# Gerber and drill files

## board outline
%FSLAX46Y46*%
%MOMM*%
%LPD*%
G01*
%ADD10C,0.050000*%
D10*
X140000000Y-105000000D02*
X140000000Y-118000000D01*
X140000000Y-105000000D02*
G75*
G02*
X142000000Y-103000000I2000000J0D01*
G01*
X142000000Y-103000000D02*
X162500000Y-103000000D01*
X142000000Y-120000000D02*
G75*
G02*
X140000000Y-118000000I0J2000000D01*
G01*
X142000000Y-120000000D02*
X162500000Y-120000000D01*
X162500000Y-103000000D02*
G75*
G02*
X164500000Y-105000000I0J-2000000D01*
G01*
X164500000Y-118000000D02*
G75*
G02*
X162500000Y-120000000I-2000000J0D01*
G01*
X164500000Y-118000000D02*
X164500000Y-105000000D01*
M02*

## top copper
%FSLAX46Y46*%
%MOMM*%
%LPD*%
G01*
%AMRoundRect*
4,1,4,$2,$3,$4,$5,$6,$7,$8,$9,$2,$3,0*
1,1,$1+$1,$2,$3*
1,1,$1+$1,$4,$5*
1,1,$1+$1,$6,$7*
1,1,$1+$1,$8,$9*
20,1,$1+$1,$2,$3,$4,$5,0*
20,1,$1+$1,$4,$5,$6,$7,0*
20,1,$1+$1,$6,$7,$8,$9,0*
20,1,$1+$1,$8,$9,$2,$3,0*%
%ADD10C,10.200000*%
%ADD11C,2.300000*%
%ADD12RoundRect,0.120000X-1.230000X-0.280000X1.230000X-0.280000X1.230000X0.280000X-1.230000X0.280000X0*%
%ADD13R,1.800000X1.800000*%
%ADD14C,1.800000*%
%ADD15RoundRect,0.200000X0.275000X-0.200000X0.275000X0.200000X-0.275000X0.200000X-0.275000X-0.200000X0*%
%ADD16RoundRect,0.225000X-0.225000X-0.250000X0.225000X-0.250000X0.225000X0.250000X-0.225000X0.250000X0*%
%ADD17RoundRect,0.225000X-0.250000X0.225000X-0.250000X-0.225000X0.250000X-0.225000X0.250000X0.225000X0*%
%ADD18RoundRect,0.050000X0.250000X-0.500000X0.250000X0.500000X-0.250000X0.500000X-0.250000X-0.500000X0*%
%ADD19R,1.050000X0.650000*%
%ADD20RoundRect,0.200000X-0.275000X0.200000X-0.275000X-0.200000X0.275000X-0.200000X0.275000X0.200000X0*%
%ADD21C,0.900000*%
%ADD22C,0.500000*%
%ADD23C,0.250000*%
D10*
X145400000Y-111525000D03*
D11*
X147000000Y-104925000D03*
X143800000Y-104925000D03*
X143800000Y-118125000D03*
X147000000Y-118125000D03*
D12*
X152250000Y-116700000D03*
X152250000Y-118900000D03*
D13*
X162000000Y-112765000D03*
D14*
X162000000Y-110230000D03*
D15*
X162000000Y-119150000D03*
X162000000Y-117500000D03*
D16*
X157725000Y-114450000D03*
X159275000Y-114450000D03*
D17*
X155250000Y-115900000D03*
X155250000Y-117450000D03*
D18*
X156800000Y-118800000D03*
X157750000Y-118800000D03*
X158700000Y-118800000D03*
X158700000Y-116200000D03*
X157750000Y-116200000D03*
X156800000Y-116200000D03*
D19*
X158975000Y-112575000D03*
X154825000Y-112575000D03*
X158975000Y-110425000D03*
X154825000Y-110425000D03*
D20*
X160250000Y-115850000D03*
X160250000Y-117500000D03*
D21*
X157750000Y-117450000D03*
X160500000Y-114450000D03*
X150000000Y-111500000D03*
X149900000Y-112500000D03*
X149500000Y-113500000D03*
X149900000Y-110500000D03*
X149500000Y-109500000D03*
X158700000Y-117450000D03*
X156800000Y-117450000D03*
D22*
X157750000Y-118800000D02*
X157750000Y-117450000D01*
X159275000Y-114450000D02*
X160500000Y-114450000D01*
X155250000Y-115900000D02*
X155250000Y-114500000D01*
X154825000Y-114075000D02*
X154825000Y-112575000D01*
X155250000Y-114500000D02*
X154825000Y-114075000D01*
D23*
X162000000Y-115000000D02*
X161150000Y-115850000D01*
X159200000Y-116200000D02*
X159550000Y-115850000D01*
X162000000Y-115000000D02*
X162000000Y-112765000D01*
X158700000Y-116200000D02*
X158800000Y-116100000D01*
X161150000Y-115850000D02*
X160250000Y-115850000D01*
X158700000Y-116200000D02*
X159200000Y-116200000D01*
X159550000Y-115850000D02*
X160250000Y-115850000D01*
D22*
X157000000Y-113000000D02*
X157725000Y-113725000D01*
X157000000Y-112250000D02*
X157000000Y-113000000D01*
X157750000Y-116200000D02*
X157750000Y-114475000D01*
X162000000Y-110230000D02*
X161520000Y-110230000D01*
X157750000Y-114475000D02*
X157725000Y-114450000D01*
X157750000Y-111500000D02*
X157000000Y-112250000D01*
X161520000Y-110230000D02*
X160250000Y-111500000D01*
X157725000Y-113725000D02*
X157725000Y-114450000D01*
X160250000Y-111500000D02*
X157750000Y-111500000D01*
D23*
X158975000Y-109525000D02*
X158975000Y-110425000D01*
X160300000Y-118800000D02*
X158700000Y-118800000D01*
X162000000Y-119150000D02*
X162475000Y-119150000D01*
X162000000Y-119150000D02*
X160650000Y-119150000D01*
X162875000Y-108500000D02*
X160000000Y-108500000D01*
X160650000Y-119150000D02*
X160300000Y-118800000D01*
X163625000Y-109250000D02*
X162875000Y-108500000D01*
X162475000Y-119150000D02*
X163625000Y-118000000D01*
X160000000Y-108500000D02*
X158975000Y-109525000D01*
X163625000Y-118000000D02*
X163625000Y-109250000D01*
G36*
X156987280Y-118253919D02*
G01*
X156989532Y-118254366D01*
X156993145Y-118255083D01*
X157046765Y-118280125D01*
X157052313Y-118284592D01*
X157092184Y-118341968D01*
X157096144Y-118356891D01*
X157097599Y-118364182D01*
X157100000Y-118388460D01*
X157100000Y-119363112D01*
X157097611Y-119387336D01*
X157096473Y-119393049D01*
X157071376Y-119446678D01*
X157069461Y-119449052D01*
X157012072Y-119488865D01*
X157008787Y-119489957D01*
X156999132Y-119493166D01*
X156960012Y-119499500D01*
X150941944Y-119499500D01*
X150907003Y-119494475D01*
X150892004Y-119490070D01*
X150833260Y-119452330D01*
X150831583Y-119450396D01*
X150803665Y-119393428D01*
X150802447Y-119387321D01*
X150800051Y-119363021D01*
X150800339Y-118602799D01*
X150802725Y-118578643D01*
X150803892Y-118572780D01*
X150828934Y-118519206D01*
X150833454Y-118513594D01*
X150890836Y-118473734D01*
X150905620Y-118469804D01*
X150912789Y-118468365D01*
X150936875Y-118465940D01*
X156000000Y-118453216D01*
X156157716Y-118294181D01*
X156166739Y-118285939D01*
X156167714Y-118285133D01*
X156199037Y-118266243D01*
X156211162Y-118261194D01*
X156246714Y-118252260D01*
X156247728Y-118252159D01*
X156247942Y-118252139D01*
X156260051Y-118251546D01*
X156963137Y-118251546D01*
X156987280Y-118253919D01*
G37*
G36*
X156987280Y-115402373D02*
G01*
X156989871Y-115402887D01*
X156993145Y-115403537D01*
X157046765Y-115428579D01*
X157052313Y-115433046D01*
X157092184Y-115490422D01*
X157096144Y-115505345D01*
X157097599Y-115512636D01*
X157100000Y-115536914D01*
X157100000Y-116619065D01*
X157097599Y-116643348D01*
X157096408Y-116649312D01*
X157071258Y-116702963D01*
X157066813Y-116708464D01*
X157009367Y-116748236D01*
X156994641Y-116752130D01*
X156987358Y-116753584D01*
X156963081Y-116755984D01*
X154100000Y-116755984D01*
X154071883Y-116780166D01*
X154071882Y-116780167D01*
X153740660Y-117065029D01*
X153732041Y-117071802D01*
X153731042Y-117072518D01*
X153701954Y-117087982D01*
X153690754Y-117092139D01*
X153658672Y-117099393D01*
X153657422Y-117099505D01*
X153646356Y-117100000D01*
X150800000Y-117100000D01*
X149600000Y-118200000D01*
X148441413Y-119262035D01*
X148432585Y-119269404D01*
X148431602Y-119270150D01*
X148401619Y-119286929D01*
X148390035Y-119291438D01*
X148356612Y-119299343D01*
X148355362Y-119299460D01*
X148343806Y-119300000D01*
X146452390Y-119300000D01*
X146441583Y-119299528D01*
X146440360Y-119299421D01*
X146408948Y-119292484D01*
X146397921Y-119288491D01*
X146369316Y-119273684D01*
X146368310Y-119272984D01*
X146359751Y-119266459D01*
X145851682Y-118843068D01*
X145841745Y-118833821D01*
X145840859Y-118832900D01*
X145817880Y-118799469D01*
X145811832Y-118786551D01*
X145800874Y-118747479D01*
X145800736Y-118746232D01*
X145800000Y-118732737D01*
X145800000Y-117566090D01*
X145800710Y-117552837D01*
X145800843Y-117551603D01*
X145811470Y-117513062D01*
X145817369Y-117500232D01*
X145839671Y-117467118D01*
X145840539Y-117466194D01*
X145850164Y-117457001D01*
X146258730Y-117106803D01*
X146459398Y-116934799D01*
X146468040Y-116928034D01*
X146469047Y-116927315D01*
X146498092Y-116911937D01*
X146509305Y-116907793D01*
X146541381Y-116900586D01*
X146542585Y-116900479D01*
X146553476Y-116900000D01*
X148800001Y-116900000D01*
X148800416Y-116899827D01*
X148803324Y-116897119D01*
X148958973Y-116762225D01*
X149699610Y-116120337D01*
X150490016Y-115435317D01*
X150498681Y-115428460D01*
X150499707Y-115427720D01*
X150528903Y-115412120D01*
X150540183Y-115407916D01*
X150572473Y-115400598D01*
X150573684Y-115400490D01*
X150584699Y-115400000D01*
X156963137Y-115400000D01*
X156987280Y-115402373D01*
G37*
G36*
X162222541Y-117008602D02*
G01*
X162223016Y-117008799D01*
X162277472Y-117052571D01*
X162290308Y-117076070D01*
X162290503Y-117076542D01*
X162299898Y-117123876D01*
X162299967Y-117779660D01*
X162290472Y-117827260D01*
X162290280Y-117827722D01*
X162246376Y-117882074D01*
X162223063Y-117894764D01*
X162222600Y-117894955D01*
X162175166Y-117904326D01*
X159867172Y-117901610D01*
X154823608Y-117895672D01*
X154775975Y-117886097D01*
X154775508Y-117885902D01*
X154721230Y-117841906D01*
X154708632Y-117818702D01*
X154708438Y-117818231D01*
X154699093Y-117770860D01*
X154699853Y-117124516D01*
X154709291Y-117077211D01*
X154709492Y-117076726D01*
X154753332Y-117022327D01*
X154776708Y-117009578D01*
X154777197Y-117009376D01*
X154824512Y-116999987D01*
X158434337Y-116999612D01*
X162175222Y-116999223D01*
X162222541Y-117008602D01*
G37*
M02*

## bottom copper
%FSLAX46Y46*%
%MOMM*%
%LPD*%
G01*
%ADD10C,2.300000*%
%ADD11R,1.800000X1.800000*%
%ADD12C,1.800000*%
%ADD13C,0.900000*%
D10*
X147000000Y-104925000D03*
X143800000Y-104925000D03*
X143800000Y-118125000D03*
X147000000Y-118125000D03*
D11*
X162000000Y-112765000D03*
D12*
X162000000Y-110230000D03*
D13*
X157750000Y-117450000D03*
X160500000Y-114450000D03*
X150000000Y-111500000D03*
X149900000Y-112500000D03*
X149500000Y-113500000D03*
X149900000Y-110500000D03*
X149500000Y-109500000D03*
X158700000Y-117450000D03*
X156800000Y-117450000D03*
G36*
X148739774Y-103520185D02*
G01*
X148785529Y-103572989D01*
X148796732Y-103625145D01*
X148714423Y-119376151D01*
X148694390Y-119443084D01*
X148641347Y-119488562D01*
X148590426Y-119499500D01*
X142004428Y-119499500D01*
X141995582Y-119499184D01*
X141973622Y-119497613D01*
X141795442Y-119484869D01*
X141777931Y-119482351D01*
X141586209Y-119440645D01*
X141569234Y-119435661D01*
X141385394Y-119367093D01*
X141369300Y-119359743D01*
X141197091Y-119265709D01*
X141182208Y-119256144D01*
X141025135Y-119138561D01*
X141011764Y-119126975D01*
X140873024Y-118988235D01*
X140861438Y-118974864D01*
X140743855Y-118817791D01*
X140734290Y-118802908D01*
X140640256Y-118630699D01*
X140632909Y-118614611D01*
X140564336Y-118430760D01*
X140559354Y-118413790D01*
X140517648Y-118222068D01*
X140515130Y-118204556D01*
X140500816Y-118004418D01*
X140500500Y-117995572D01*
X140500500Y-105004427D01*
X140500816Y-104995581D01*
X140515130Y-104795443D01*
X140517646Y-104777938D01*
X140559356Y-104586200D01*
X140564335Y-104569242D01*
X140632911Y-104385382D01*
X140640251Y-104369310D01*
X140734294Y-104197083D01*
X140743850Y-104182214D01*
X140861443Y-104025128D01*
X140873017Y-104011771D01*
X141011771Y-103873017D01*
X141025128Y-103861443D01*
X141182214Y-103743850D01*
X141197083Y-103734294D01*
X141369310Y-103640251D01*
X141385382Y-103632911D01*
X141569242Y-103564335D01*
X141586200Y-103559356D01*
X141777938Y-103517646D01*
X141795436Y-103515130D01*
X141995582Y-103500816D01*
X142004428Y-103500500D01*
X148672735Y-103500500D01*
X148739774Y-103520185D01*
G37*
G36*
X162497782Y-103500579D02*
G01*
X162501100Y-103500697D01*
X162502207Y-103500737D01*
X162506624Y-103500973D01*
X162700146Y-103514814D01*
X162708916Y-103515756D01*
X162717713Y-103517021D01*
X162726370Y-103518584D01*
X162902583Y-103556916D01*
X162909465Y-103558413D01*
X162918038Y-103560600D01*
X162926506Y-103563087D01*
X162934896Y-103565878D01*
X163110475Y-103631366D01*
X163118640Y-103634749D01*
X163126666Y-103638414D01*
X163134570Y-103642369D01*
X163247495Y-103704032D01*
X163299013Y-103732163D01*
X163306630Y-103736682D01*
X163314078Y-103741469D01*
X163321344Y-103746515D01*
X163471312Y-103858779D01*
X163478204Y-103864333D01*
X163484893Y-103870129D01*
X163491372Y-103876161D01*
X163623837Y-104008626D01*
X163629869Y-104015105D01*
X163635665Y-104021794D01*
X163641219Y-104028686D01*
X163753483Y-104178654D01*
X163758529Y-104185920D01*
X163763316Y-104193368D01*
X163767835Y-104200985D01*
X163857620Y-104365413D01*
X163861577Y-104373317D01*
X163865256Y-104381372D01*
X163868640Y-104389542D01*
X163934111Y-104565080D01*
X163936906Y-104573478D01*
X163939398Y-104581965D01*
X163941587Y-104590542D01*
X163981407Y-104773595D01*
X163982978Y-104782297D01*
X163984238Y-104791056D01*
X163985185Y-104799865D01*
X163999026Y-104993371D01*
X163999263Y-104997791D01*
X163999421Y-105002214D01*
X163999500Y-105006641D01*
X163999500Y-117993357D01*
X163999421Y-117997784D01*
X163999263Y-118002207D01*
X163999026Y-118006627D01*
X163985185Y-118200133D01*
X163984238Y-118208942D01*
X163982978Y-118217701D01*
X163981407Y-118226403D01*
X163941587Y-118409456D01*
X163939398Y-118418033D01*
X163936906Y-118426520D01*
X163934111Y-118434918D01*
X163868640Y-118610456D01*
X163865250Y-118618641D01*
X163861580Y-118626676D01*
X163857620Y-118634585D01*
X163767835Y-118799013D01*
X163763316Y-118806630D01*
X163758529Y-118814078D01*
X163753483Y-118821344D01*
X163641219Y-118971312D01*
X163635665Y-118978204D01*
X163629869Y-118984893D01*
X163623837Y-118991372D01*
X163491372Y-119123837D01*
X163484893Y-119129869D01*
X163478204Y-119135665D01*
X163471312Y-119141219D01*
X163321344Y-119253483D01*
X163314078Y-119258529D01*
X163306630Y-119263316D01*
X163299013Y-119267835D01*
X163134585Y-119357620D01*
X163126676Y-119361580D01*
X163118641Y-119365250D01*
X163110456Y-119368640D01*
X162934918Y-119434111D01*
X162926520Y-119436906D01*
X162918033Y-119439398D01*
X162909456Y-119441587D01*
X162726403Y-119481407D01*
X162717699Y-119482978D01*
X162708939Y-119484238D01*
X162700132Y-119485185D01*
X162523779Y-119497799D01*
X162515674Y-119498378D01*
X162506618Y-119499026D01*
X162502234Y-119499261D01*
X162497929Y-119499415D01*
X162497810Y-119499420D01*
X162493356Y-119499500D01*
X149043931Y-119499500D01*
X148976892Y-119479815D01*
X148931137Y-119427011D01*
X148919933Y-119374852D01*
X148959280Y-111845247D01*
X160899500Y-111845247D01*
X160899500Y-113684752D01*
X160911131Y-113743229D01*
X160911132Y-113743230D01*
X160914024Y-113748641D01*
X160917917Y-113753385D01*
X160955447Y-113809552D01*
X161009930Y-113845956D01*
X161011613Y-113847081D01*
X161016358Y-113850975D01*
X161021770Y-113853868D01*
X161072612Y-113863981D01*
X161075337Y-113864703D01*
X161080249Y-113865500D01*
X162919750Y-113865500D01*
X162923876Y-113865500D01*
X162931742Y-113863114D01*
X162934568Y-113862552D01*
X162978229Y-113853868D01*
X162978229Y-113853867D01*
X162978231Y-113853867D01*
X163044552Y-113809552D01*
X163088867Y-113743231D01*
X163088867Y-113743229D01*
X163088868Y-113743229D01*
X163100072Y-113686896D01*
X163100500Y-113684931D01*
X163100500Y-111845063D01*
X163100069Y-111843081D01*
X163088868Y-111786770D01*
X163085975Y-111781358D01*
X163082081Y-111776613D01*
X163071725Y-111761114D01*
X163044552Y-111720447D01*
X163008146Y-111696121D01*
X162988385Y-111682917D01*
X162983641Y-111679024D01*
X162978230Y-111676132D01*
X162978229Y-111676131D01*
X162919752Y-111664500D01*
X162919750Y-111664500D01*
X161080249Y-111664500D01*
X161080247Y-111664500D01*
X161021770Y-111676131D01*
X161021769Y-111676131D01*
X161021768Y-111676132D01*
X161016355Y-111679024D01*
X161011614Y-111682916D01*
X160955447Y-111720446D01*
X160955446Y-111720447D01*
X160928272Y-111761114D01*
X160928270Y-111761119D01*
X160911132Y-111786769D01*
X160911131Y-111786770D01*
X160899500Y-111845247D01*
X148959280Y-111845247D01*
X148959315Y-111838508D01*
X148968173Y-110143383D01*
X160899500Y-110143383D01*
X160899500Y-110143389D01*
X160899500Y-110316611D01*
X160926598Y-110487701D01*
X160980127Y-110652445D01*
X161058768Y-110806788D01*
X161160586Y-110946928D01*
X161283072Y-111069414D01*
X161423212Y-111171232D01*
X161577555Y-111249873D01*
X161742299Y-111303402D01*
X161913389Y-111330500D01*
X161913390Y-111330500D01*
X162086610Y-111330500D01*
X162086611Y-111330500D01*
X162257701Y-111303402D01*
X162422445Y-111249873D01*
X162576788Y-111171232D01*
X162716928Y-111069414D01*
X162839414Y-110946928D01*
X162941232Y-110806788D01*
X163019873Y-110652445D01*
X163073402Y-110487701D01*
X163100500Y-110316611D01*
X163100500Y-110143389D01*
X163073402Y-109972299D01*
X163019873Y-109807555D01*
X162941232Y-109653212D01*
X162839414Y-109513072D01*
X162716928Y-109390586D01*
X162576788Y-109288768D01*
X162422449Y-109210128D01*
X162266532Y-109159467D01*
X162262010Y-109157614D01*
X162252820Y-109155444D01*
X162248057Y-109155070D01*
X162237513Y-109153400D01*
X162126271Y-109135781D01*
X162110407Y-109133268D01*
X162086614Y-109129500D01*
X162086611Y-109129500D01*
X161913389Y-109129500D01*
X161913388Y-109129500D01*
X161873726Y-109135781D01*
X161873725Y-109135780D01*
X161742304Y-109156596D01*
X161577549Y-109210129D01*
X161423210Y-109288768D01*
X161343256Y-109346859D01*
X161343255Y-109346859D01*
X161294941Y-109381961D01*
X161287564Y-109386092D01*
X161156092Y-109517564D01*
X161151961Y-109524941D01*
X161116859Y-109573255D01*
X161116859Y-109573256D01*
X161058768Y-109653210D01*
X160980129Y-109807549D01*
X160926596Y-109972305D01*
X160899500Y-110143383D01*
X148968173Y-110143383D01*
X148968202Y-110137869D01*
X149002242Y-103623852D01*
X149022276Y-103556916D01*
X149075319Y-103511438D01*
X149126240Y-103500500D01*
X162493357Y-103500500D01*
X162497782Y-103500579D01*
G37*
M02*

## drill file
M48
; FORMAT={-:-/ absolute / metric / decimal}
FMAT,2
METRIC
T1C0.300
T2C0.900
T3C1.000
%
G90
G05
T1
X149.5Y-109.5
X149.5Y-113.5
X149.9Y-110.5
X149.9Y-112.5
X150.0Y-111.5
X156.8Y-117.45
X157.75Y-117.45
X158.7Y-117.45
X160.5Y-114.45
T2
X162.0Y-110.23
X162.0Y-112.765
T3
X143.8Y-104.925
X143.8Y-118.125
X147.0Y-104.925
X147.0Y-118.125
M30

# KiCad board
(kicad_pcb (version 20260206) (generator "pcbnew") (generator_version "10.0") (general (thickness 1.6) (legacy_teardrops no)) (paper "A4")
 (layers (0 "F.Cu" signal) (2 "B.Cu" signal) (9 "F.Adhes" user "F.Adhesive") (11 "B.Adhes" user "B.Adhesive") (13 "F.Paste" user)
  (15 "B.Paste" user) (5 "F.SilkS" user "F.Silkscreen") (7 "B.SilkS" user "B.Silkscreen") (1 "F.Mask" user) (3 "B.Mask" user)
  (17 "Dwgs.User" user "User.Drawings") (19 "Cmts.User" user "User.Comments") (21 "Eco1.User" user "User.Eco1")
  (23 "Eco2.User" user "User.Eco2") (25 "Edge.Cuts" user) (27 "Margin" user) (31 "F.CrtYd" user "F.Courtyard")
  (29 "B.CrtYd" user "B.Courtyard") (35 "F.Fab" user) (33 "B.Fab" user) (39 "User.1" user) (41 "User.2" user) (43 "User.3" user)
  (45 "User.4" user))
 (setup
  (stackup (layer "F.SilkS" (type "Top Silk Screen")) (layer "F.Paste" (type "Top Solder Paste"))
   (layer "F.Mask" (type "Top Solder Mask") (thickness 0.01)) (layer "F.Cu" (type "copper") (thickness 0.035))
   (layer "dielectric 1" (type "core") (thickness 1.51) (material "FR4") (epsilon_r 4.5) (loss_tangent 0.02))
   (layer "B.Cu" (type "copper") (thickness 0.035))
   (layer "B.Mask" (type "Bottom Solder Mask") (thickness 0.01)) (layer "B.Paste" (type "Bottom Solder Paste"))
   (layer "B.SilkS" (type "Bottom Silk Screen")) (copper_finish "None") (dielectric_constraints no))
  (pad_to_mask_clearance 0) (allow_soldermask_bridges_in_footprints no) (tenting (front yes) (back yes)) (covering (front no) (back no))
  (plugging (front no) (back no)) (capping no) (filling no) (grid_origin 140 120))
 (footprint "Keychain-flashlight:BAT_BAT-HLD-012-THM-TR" (layer "F.Cu") (at 145.4 111.525 -90)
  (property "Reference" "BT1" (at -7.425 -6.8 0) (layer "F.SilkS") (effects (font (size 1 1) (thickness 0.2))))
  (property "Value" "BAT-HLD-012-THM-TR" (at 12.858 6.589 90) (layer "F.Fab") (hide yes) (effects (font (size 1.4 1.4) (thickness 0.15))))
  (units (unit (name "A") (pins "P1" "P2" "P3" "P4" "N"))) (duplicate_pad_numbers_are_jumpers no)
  (pad "N" smd circle (at 0 0 270) (size 10.2 10.2) (layers "F.Cu" "F.Mask") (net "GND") (solder_mask_margin 0.102))
  (pad "P1" thru_hole circle (at -6.6 -1.6 270) (size 2.3 2.3) (drill 1) (layers "*.Cu" "*.Mask") (remove_unused_layers no) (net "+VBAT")
   (solder_mask_margin 0.102))
  (pad "P2" thru_hole circle (at -6.6 1.6 270) (size 2.3 2.3) (drill 1) (layers "*.Cu" "*.Mask") (remove_unused_layers no) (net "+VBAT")
   (solder_mask_margin 0.102))
  (pad "P3" thru_hole circle (at 6.6 1.6 270) (size 2.3 2.3) (drill 1) (layers "*.Cu" "*.Mask") (remove_unused_layers no) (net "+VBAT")
   (solder_mask_margin 0.102))
  (pad "P4" thru_hole circle (at 6.6 -1.6 270) (size 2.3 2.3) (drill 1) (layers "*.Cu" "*.Mask") (remove_unused_layers no) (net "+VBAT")
   (solder_mask_margin 0.102)))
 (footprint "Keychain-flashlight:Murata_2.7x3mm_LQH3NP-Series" (layer "F.Cu") (at 152.25 117.8 -90)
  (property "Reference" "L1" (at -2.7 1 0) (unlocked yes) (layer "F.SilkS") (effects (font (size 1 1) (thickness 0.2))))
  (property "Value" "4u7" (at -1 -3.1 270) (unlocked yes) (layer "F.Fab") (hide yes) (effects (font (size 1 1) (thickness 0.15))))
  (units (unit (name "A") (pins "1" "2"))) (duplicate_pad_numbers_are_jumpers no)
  (pad "1" smd roundrect (at -1.1 0) (size 2.7 0.8) (layers "F.Cu" "F.Mask" "F.Paste") (roundrect_rratio 0.15) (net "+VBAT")
   (thermal_bridge_angle 45))
  (pad "2" smd roundrect (at 1.1 0) (size 2.7 0.8) (layers "F.Cu" "F.Mask" "F.Paste") (roundrect_rratio 0.15) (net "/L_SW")
   (thermal_bridge_angle 45)))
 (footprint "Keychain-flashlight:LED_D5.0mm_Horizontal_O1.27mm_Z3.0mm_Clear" (layer "F.Cu") (at 162 112.77 90)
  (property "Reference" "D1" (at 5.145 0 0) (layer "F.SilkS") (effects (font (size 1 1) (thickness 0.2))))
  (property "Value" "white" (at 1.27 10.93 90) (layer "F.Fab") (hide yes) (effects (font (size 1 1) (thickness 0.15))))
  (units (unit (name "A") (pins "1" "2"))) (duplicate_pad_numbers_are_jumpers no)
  (pad "1" thru_hole rect (at 0.005 0 90) (size 1.8 1.8) (drill 0.9) (layers "*.Cu" "*.Mask") (remove_unused_layers no) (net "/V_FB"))
  (pad "2" thru_hole circle (at 2.54 0 90) (size 1.8 1.8) (drill 0.9) (layers "*.Cu" "*.Mask") (remove_unused_layers no) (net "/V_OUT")))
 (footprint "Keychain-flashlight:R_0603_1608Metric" (layer "F.Cu") (at 162 118.325 90)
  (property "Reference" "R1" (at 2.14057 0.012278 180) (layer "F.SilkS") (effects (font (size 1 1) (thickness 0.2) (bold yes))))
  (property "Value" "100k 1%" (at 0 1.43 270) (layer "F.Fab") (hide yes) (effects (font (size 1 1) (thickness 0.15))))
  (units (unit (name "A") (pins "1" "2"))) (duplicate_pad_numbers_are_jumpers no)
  (pad "1" smd roundrect (at -0.825 0 90) (size 0.8 0.95) (layers "F.Cu" "F.Mask" "F.Paste") (roundrect_rratio 0.25) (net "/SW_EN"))
  (pad "2" smd roundrect (at 0.825 0 90) (size 0.8 0.95) (layers "F.Cu" "F.Mask" "F.Paste") (roundrect_rratio 0.25) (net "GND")))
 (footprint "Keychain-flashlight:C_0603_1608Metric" (layer "F.Cu") (at 158.5 114.45)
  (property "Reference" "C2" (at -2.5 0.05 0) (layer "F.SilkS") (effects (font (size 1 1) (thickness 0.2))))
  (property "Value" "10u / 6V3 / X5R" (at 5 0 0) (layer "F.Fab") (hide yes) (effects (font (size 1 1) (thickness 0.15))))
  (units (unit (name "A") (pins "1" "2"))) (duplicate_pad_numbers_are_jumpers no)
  (pad "1" smd roundrect (at -0.775 0) (size 0.9 0.95) (layers "F.Cu" "F.Mask" "F.Paste") (roundrect_rratio 0.25) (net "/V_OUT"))
  (pad "2" smd roundrect (at 0.775 0) (size 0.9 0.95) (layers "F.Cu" "F.Mask" "F.Paste") (roundrect_rratio 0.25) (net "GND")))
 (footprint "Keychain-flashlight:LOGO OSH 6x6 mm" (layer "F.Cu") (at 157.498962 106.370917)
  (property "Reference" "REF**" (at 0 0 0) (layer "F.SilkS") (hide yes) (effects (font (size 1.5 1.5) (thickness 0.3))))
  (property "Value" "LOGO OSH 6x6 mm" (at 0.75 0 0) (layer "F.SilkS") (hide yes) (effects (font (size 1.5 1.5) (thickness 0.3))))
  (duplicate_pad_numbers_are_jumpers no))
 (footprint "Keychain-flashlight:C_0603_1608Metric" (layer "F.Cu") (at 155.25 116.675 -90)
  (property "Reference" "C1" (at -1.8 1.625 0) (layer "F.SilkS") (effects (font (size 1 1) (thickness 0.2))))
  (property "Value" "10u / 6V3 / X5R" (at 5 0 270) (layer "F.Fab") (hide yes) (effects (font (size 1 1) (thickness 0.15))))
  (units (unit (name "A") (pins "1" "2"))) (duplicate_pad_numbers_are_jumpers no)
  (pad "1" smd roundrect (at -0.775 0 270) (size 0.9 0.95) (layers "F.Cu" "F.Mask" "F.Paste") (roundrect_rratio 0.25) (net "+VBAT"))
  (pad "2" smd roundrect (at 0.775 0 270) (size 0.9 0.95) (layers "F.Cu" "F.Mask" "F.Paste") (roundrect_rratio 0.25) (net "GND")))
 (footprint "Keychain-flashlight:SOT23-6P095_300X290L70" (layer "F.Cu") (at 157.75 117.5 90)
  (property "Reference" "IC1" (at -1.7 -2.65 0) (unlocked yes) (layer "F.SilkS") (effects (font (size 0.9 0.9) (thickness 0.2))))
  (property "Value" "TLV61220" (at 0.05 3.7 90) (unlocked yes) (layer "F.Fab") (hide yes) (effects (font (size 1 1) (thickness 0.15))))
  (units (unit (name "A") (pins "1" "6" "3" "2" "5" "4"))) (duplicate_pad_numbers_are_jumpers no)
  (pad "1" smd roundrect (at -1.3 -0.95 90) (size 1.1 0.6) (layers "F.Cu" "F.Mask" "F.Paste") (roundrect_rratio 0.08333333333) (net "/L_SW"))
  (pad "2" smd roundrect (at -1.3 0 90) (size 1.1 0.6) (layers "F.Cu" "F.Mask" "F.Paste") (roundrect_rratio 0.08333333333) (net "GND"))
  (pad "3" smd roundrect (at -1.3 0.95 90) (size 1.1 0.6) (layers "F.Cu" "F.Mask" "F.Paste") (roundrect_rratio 0.08333333333) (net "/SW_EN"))
  (pad "4" smd roundrect (at 1.3 0.95 90) (size 1.1 0.6) (layers "F.Cu" "F.Mask" "F.Paste") (roundrect_rratio 0.08333333333) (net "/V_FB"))
  (pad "5" smd roundrect (at 1.3 0 90) (size 1.1 0.6) (layers "F.Cu" "F.Mask" "F.Paste") (roundrect_rratio 0.08333333333) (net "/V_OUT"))
  (pad "6" smd roundrect (at 1.3 -0.95 90) (size 1.1 0.6) (layers "F.Cu" "F.Mask" "F.Paste") (roundrect_rratio 0.08333333333) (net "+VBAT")))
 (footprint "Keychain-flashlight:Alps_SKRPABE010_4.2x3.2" (layer "F.Cu") (at 156.9 111.5 180)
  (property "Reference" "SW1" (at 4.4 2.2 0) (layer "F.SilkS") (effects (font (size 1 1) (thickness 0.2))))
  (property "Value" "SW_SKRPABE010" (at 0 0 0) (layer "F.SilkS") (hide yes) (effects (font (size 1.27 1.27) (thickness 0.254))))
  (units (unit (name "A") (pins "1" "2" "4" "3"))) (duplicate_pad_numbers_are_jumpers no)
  (pad "1" smd rect (at -2.075 -1.075 270) (size 0.65 1.05) (layers "F.Cu" "F.Mask" "F.Paste") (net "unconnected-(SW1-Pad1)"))
  (pad "2" smd rect (at 2.075 -1.075 270) (size 0.65 1.05) (layers "F.Cu" "F.Mask" "F.Paste") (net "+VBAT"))
  (pad "3" smd rect (at -2.075 1.075 270) (size 0.65 1.05) (layers "F.Cu" "F.Mask" "F.Paste") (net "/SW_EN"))
  (pad "4" smd rect (at 2.075 1.075 270) (size 0.65 1.05) (layers "F.Cu" "F.Mask" "F.Paste") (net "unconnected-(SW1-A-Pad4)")))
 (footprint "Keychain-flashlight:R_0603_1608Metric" (layer "F.Cu") (at 160.25 116.675 -90)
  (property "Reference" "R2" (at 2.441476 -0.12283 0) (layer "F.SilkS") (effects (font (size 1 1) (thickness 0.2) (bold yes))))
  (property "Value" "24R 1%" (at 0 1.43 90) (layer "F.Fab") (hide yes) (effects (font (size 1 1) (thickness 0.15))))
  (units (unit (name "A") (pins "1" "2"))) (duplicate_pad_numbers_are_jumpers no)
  (pad "1" smd roundrect (at -0.825 0 270) (size 0.8 0.95) (layers "F.Cu" "F.Mask" "F.Paste") (roundrect_rratio 0.25) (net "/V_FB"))
  (pad "2" smd roundrect (at 0.825 0 270) (size 0.8 0.95) (layers "F.Cu" "F.Mask" "F.Paste") (roundrect_rratio 0.25) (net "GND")))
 (gr_line (start 140 105) (end 140 118) (stroke (width 0.05) (type default)) (layer "Edge.Cuts"))
 (gr_arc (start 140 105) (mid 140.585786 103.585786) (end 142 103) (stroke (width 0.05) (type default)) (layer "Edge.Cuts"))
 (gr_line (start 142 103) (end 162.5 103) (stroke (width 0.05) (type default)) (layer "Edge.Cuts"))
 (gr_arc (start 142 120) (mid 140.585786 119.414214) (end 140 118) (stroke (width 0.05) (type default)) (layer "Edge.Cuts"))
 (gr_line (start 142 120) (end 162.5 120) (stroke (width 0.05) (type default)) (layer "Edge.Cuts"))
 (gr_arc (start 162.5 103) (mid 163.914214 103.585786) (end 164.5 105) (stroke (width 0.05) (type default)) (layer "Edge.Cuts"))
 (gr_arc (start 164.5 118) (mid 163.914214 119.414214) (end 162.5 120) (stroke (width 0.05) (type default)) (layer "Edge.Cuts"))
 (gr_line (start 164.5 118) (end 164.5 105) (stroke (width 0.05) (type default)) (layer "Edge.Cuts"))
 (segment (start 157.75 118.8) (end 157.75 117.45) (width 0.5) (layer "F.Cu") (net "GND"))
 (segment (start 159.275 114.45) (end 160.5 114.45) (width 0.5) (layer "F.Cu") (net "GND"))
 (via (at 157.75 117.45) (size 0.9) (drill 0.3) (layers "F.Cu" "B.Cu") (free yes) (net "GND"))
 (via (at 160.5 114.45) (size 0.9) (drill 0.3) (layers "F.Cu" "B.Cu") (free yes) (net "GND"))
 (via (at 150 111.5) (size 0.9) (drill 0.3) (layers "F.Cu" "B.Cu") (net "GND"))
 (via (at 149.9 112.5) (size 0.9) (drill 0.3) (layers "F.Cu" "B.Cu") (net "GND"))
 (via (at 149.5 113.5) (size 0.9) (drill 0.3) (layers "F.Cu" "B.Cu") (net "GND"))
 (via (at 149.9 110.5) (size 0.9) (drill 0.3) (layers "F.Cu" "B.Cu") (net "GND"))
 (via (at 149.5 109.5) (size 0.9) (drill 0.3) (layers "F.Cu" "B.Cu") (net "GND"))
 (via (at 158.7 117.45) (size 0.9) (drill 0.3) (layers "F.Cu" "B.Cu") (free yes) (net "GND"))
 (via (at 156.8 117.45) (size 0.9) (drill 0.3) (layers "F.Cu" "B.Cu") (free yes) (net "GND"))
 (segment (start 155.25 115.9) (end 155.25 114.5) (width 0.5) (layer "F.Cu") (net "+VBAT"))
 (segment (start 154.825 114.075) (end 154.825 112.575) (width 0.5) (layer "F.Cu") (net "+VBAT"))
 (segment (start 155.25 114.5) (end 154.825 114.075) (width 0.5) (layer "F.Cu") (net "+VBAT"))
 (segment (start 162 115) (end 161.15 115.85) (width 0.25) (layer "F.Cu") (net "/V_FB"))
 (segment (start 159.2 116.2) (end 159.55 115.85) (width 0.25) (layer "F.Cu") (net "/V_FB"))
 (segment (start 162 115) (end 162 112.765) (width 0.25) (layer "F.Cu") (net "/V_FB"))
 (segment (start 158.7 116.2) (end 158.8 116.1) (width 0.25) (layer "F.Cu") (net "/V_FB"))
 (segment (start 161.15 115.85) (end 160.25 115.85) (width 0.25) (layer "F.Cu") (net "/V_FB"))
 (segment (start 158.7 116.2) (end 159.2 116.2) (width 0.25) (layer "F.Cu") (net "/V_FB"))
 (segment (start 159.55 115.85) (end 160.25 115.85) (width 0.25) (layer "F.Cu") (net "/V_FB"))
 (segment (start 157 113) (end 157.725 113.725) (width 0.5) (layer "F.Cu") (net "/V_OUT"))
 (segment (start 157 112.25) (end 157 113) (width 0.5) (layer "F.Cu") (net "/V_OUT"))
 (segment (start 157.75 116.2) (end 157.75 114.475) (width 0.5) (layer "F.Cu") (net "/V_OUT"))
 (segment (start 162 110.23) (end 161.52 110.23) (width 0.5) (layer "F.Cu") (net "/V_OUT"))
 (segment (start 157.75 114.475) (end 157.725 114.45) (width 0.5) (layer "F.Cu") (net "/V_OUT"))
 (segment (start 157.75 111.5) (end 157 112.25) (width 0.5) (layer "F.Cu") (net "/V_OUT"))
 (segment (start 161.52 110.23) (end 160.25 111.5) (width 0.5) (layer "F.Cu") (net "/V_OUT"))
 (segment (start 157.725 113.725) (end 157.725 114.45) (width 0.5) (layer "F.Cu") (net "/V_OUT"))
 (segment (start 160.25 111.5) (end 157.75 111.5) (width 0.5) (layer "F.Cu") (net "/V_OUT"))
 (segment (start 158.975 109.525) (end 158.975 110.425) (width 0.25) (layer "F.Cu") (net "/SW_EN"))
 (segment (start 160.3 118.8) (end 158.7 118.8) (width 0.25) (layer "F.Cu") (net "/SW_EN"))
 (segment (start 162 119.15) (end 162.475 119.15) (width 0.25) (layer "F.Cu") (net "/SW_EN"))
 (segment (start 162 119.15) (end 160.65 119.15) (width 0.25) (layer "F.Cu") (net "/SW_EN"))
 (segment (start 162.875 108.5) (end 160 108.5) (width 0.25) (layer "F.Cu") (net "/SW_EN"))
 (segment (start 160.65 119.15) (end 160.3 118.8) (width 0.25) (layer "F.Cu") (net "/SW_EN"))
 (segment (start 163.625 109.25) (end 162.875 108.5) (width 0.25) (layer "F.Cu") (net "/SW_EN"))
 (segment (start 162.475 119.15) (end 163.625 118) (width 0.25) (layer "F.Cu") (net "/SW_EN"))
 (segment (start 160 108.5) (end 158.975 109.525) (width 0.25) (layer "F.Cu") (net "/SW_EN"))
 (segment (start 163.625 118) (end 163.625 109.25) (width 0.25) (layer "F.Cu") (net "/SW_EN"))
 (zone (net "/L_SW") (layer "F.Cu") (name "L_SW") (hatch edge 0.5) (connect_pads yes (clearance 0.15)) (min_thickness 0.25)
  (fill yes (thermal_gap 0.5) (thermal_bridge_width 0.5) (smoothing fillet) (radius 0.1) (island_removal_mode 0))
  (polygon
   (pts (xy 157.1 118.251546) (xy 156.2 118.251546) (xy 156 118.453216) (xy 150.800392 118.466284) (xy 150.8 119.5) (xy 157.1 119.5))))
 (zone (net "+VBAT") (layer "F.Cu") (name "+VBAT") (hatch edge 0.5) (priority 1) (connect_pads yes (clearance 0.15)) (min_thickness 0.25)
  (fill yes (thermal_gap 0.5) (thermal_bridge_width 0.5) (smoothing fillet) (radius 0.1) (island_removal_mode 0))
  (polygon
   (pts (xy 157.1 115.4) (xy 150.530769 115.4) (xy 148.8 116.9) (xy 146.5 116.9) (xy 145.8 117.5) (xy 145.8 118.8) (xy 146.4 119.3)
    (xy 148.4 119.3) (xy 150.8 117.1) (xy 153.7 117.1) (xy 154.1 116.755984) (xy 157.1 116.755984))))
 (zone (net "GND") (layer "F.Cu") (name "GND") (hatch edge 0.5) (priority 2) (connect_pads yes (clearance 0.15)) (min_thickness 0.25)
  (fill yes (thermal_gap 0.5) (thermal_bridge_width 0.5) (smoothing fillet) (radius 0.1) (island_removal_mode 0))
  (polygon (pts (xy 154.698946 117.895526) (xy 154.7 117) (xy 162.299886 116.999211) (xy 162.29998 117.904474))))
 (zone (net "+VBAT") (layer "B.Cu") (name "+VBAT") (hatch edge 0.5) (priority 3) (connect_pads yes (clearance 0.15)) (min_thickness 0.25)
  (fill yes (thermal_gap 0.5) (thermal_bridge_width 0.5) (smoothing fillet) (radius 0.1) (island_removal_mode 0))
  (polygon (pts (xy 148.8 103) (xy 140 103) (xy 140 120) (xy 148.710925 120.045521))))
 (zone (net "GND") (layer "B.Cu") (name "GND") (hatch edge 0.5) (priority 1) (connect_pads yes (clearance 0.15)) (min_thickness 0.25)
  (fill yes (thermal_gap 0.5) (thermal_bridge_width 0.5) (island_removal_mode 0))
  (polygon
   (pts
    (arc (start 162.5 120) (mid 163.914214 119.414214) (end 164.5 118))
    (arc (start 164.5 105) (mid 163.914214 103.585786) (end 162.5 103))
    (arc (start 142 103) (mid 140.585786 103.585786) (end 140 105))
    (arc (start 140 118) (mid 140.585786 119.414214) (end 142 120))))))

